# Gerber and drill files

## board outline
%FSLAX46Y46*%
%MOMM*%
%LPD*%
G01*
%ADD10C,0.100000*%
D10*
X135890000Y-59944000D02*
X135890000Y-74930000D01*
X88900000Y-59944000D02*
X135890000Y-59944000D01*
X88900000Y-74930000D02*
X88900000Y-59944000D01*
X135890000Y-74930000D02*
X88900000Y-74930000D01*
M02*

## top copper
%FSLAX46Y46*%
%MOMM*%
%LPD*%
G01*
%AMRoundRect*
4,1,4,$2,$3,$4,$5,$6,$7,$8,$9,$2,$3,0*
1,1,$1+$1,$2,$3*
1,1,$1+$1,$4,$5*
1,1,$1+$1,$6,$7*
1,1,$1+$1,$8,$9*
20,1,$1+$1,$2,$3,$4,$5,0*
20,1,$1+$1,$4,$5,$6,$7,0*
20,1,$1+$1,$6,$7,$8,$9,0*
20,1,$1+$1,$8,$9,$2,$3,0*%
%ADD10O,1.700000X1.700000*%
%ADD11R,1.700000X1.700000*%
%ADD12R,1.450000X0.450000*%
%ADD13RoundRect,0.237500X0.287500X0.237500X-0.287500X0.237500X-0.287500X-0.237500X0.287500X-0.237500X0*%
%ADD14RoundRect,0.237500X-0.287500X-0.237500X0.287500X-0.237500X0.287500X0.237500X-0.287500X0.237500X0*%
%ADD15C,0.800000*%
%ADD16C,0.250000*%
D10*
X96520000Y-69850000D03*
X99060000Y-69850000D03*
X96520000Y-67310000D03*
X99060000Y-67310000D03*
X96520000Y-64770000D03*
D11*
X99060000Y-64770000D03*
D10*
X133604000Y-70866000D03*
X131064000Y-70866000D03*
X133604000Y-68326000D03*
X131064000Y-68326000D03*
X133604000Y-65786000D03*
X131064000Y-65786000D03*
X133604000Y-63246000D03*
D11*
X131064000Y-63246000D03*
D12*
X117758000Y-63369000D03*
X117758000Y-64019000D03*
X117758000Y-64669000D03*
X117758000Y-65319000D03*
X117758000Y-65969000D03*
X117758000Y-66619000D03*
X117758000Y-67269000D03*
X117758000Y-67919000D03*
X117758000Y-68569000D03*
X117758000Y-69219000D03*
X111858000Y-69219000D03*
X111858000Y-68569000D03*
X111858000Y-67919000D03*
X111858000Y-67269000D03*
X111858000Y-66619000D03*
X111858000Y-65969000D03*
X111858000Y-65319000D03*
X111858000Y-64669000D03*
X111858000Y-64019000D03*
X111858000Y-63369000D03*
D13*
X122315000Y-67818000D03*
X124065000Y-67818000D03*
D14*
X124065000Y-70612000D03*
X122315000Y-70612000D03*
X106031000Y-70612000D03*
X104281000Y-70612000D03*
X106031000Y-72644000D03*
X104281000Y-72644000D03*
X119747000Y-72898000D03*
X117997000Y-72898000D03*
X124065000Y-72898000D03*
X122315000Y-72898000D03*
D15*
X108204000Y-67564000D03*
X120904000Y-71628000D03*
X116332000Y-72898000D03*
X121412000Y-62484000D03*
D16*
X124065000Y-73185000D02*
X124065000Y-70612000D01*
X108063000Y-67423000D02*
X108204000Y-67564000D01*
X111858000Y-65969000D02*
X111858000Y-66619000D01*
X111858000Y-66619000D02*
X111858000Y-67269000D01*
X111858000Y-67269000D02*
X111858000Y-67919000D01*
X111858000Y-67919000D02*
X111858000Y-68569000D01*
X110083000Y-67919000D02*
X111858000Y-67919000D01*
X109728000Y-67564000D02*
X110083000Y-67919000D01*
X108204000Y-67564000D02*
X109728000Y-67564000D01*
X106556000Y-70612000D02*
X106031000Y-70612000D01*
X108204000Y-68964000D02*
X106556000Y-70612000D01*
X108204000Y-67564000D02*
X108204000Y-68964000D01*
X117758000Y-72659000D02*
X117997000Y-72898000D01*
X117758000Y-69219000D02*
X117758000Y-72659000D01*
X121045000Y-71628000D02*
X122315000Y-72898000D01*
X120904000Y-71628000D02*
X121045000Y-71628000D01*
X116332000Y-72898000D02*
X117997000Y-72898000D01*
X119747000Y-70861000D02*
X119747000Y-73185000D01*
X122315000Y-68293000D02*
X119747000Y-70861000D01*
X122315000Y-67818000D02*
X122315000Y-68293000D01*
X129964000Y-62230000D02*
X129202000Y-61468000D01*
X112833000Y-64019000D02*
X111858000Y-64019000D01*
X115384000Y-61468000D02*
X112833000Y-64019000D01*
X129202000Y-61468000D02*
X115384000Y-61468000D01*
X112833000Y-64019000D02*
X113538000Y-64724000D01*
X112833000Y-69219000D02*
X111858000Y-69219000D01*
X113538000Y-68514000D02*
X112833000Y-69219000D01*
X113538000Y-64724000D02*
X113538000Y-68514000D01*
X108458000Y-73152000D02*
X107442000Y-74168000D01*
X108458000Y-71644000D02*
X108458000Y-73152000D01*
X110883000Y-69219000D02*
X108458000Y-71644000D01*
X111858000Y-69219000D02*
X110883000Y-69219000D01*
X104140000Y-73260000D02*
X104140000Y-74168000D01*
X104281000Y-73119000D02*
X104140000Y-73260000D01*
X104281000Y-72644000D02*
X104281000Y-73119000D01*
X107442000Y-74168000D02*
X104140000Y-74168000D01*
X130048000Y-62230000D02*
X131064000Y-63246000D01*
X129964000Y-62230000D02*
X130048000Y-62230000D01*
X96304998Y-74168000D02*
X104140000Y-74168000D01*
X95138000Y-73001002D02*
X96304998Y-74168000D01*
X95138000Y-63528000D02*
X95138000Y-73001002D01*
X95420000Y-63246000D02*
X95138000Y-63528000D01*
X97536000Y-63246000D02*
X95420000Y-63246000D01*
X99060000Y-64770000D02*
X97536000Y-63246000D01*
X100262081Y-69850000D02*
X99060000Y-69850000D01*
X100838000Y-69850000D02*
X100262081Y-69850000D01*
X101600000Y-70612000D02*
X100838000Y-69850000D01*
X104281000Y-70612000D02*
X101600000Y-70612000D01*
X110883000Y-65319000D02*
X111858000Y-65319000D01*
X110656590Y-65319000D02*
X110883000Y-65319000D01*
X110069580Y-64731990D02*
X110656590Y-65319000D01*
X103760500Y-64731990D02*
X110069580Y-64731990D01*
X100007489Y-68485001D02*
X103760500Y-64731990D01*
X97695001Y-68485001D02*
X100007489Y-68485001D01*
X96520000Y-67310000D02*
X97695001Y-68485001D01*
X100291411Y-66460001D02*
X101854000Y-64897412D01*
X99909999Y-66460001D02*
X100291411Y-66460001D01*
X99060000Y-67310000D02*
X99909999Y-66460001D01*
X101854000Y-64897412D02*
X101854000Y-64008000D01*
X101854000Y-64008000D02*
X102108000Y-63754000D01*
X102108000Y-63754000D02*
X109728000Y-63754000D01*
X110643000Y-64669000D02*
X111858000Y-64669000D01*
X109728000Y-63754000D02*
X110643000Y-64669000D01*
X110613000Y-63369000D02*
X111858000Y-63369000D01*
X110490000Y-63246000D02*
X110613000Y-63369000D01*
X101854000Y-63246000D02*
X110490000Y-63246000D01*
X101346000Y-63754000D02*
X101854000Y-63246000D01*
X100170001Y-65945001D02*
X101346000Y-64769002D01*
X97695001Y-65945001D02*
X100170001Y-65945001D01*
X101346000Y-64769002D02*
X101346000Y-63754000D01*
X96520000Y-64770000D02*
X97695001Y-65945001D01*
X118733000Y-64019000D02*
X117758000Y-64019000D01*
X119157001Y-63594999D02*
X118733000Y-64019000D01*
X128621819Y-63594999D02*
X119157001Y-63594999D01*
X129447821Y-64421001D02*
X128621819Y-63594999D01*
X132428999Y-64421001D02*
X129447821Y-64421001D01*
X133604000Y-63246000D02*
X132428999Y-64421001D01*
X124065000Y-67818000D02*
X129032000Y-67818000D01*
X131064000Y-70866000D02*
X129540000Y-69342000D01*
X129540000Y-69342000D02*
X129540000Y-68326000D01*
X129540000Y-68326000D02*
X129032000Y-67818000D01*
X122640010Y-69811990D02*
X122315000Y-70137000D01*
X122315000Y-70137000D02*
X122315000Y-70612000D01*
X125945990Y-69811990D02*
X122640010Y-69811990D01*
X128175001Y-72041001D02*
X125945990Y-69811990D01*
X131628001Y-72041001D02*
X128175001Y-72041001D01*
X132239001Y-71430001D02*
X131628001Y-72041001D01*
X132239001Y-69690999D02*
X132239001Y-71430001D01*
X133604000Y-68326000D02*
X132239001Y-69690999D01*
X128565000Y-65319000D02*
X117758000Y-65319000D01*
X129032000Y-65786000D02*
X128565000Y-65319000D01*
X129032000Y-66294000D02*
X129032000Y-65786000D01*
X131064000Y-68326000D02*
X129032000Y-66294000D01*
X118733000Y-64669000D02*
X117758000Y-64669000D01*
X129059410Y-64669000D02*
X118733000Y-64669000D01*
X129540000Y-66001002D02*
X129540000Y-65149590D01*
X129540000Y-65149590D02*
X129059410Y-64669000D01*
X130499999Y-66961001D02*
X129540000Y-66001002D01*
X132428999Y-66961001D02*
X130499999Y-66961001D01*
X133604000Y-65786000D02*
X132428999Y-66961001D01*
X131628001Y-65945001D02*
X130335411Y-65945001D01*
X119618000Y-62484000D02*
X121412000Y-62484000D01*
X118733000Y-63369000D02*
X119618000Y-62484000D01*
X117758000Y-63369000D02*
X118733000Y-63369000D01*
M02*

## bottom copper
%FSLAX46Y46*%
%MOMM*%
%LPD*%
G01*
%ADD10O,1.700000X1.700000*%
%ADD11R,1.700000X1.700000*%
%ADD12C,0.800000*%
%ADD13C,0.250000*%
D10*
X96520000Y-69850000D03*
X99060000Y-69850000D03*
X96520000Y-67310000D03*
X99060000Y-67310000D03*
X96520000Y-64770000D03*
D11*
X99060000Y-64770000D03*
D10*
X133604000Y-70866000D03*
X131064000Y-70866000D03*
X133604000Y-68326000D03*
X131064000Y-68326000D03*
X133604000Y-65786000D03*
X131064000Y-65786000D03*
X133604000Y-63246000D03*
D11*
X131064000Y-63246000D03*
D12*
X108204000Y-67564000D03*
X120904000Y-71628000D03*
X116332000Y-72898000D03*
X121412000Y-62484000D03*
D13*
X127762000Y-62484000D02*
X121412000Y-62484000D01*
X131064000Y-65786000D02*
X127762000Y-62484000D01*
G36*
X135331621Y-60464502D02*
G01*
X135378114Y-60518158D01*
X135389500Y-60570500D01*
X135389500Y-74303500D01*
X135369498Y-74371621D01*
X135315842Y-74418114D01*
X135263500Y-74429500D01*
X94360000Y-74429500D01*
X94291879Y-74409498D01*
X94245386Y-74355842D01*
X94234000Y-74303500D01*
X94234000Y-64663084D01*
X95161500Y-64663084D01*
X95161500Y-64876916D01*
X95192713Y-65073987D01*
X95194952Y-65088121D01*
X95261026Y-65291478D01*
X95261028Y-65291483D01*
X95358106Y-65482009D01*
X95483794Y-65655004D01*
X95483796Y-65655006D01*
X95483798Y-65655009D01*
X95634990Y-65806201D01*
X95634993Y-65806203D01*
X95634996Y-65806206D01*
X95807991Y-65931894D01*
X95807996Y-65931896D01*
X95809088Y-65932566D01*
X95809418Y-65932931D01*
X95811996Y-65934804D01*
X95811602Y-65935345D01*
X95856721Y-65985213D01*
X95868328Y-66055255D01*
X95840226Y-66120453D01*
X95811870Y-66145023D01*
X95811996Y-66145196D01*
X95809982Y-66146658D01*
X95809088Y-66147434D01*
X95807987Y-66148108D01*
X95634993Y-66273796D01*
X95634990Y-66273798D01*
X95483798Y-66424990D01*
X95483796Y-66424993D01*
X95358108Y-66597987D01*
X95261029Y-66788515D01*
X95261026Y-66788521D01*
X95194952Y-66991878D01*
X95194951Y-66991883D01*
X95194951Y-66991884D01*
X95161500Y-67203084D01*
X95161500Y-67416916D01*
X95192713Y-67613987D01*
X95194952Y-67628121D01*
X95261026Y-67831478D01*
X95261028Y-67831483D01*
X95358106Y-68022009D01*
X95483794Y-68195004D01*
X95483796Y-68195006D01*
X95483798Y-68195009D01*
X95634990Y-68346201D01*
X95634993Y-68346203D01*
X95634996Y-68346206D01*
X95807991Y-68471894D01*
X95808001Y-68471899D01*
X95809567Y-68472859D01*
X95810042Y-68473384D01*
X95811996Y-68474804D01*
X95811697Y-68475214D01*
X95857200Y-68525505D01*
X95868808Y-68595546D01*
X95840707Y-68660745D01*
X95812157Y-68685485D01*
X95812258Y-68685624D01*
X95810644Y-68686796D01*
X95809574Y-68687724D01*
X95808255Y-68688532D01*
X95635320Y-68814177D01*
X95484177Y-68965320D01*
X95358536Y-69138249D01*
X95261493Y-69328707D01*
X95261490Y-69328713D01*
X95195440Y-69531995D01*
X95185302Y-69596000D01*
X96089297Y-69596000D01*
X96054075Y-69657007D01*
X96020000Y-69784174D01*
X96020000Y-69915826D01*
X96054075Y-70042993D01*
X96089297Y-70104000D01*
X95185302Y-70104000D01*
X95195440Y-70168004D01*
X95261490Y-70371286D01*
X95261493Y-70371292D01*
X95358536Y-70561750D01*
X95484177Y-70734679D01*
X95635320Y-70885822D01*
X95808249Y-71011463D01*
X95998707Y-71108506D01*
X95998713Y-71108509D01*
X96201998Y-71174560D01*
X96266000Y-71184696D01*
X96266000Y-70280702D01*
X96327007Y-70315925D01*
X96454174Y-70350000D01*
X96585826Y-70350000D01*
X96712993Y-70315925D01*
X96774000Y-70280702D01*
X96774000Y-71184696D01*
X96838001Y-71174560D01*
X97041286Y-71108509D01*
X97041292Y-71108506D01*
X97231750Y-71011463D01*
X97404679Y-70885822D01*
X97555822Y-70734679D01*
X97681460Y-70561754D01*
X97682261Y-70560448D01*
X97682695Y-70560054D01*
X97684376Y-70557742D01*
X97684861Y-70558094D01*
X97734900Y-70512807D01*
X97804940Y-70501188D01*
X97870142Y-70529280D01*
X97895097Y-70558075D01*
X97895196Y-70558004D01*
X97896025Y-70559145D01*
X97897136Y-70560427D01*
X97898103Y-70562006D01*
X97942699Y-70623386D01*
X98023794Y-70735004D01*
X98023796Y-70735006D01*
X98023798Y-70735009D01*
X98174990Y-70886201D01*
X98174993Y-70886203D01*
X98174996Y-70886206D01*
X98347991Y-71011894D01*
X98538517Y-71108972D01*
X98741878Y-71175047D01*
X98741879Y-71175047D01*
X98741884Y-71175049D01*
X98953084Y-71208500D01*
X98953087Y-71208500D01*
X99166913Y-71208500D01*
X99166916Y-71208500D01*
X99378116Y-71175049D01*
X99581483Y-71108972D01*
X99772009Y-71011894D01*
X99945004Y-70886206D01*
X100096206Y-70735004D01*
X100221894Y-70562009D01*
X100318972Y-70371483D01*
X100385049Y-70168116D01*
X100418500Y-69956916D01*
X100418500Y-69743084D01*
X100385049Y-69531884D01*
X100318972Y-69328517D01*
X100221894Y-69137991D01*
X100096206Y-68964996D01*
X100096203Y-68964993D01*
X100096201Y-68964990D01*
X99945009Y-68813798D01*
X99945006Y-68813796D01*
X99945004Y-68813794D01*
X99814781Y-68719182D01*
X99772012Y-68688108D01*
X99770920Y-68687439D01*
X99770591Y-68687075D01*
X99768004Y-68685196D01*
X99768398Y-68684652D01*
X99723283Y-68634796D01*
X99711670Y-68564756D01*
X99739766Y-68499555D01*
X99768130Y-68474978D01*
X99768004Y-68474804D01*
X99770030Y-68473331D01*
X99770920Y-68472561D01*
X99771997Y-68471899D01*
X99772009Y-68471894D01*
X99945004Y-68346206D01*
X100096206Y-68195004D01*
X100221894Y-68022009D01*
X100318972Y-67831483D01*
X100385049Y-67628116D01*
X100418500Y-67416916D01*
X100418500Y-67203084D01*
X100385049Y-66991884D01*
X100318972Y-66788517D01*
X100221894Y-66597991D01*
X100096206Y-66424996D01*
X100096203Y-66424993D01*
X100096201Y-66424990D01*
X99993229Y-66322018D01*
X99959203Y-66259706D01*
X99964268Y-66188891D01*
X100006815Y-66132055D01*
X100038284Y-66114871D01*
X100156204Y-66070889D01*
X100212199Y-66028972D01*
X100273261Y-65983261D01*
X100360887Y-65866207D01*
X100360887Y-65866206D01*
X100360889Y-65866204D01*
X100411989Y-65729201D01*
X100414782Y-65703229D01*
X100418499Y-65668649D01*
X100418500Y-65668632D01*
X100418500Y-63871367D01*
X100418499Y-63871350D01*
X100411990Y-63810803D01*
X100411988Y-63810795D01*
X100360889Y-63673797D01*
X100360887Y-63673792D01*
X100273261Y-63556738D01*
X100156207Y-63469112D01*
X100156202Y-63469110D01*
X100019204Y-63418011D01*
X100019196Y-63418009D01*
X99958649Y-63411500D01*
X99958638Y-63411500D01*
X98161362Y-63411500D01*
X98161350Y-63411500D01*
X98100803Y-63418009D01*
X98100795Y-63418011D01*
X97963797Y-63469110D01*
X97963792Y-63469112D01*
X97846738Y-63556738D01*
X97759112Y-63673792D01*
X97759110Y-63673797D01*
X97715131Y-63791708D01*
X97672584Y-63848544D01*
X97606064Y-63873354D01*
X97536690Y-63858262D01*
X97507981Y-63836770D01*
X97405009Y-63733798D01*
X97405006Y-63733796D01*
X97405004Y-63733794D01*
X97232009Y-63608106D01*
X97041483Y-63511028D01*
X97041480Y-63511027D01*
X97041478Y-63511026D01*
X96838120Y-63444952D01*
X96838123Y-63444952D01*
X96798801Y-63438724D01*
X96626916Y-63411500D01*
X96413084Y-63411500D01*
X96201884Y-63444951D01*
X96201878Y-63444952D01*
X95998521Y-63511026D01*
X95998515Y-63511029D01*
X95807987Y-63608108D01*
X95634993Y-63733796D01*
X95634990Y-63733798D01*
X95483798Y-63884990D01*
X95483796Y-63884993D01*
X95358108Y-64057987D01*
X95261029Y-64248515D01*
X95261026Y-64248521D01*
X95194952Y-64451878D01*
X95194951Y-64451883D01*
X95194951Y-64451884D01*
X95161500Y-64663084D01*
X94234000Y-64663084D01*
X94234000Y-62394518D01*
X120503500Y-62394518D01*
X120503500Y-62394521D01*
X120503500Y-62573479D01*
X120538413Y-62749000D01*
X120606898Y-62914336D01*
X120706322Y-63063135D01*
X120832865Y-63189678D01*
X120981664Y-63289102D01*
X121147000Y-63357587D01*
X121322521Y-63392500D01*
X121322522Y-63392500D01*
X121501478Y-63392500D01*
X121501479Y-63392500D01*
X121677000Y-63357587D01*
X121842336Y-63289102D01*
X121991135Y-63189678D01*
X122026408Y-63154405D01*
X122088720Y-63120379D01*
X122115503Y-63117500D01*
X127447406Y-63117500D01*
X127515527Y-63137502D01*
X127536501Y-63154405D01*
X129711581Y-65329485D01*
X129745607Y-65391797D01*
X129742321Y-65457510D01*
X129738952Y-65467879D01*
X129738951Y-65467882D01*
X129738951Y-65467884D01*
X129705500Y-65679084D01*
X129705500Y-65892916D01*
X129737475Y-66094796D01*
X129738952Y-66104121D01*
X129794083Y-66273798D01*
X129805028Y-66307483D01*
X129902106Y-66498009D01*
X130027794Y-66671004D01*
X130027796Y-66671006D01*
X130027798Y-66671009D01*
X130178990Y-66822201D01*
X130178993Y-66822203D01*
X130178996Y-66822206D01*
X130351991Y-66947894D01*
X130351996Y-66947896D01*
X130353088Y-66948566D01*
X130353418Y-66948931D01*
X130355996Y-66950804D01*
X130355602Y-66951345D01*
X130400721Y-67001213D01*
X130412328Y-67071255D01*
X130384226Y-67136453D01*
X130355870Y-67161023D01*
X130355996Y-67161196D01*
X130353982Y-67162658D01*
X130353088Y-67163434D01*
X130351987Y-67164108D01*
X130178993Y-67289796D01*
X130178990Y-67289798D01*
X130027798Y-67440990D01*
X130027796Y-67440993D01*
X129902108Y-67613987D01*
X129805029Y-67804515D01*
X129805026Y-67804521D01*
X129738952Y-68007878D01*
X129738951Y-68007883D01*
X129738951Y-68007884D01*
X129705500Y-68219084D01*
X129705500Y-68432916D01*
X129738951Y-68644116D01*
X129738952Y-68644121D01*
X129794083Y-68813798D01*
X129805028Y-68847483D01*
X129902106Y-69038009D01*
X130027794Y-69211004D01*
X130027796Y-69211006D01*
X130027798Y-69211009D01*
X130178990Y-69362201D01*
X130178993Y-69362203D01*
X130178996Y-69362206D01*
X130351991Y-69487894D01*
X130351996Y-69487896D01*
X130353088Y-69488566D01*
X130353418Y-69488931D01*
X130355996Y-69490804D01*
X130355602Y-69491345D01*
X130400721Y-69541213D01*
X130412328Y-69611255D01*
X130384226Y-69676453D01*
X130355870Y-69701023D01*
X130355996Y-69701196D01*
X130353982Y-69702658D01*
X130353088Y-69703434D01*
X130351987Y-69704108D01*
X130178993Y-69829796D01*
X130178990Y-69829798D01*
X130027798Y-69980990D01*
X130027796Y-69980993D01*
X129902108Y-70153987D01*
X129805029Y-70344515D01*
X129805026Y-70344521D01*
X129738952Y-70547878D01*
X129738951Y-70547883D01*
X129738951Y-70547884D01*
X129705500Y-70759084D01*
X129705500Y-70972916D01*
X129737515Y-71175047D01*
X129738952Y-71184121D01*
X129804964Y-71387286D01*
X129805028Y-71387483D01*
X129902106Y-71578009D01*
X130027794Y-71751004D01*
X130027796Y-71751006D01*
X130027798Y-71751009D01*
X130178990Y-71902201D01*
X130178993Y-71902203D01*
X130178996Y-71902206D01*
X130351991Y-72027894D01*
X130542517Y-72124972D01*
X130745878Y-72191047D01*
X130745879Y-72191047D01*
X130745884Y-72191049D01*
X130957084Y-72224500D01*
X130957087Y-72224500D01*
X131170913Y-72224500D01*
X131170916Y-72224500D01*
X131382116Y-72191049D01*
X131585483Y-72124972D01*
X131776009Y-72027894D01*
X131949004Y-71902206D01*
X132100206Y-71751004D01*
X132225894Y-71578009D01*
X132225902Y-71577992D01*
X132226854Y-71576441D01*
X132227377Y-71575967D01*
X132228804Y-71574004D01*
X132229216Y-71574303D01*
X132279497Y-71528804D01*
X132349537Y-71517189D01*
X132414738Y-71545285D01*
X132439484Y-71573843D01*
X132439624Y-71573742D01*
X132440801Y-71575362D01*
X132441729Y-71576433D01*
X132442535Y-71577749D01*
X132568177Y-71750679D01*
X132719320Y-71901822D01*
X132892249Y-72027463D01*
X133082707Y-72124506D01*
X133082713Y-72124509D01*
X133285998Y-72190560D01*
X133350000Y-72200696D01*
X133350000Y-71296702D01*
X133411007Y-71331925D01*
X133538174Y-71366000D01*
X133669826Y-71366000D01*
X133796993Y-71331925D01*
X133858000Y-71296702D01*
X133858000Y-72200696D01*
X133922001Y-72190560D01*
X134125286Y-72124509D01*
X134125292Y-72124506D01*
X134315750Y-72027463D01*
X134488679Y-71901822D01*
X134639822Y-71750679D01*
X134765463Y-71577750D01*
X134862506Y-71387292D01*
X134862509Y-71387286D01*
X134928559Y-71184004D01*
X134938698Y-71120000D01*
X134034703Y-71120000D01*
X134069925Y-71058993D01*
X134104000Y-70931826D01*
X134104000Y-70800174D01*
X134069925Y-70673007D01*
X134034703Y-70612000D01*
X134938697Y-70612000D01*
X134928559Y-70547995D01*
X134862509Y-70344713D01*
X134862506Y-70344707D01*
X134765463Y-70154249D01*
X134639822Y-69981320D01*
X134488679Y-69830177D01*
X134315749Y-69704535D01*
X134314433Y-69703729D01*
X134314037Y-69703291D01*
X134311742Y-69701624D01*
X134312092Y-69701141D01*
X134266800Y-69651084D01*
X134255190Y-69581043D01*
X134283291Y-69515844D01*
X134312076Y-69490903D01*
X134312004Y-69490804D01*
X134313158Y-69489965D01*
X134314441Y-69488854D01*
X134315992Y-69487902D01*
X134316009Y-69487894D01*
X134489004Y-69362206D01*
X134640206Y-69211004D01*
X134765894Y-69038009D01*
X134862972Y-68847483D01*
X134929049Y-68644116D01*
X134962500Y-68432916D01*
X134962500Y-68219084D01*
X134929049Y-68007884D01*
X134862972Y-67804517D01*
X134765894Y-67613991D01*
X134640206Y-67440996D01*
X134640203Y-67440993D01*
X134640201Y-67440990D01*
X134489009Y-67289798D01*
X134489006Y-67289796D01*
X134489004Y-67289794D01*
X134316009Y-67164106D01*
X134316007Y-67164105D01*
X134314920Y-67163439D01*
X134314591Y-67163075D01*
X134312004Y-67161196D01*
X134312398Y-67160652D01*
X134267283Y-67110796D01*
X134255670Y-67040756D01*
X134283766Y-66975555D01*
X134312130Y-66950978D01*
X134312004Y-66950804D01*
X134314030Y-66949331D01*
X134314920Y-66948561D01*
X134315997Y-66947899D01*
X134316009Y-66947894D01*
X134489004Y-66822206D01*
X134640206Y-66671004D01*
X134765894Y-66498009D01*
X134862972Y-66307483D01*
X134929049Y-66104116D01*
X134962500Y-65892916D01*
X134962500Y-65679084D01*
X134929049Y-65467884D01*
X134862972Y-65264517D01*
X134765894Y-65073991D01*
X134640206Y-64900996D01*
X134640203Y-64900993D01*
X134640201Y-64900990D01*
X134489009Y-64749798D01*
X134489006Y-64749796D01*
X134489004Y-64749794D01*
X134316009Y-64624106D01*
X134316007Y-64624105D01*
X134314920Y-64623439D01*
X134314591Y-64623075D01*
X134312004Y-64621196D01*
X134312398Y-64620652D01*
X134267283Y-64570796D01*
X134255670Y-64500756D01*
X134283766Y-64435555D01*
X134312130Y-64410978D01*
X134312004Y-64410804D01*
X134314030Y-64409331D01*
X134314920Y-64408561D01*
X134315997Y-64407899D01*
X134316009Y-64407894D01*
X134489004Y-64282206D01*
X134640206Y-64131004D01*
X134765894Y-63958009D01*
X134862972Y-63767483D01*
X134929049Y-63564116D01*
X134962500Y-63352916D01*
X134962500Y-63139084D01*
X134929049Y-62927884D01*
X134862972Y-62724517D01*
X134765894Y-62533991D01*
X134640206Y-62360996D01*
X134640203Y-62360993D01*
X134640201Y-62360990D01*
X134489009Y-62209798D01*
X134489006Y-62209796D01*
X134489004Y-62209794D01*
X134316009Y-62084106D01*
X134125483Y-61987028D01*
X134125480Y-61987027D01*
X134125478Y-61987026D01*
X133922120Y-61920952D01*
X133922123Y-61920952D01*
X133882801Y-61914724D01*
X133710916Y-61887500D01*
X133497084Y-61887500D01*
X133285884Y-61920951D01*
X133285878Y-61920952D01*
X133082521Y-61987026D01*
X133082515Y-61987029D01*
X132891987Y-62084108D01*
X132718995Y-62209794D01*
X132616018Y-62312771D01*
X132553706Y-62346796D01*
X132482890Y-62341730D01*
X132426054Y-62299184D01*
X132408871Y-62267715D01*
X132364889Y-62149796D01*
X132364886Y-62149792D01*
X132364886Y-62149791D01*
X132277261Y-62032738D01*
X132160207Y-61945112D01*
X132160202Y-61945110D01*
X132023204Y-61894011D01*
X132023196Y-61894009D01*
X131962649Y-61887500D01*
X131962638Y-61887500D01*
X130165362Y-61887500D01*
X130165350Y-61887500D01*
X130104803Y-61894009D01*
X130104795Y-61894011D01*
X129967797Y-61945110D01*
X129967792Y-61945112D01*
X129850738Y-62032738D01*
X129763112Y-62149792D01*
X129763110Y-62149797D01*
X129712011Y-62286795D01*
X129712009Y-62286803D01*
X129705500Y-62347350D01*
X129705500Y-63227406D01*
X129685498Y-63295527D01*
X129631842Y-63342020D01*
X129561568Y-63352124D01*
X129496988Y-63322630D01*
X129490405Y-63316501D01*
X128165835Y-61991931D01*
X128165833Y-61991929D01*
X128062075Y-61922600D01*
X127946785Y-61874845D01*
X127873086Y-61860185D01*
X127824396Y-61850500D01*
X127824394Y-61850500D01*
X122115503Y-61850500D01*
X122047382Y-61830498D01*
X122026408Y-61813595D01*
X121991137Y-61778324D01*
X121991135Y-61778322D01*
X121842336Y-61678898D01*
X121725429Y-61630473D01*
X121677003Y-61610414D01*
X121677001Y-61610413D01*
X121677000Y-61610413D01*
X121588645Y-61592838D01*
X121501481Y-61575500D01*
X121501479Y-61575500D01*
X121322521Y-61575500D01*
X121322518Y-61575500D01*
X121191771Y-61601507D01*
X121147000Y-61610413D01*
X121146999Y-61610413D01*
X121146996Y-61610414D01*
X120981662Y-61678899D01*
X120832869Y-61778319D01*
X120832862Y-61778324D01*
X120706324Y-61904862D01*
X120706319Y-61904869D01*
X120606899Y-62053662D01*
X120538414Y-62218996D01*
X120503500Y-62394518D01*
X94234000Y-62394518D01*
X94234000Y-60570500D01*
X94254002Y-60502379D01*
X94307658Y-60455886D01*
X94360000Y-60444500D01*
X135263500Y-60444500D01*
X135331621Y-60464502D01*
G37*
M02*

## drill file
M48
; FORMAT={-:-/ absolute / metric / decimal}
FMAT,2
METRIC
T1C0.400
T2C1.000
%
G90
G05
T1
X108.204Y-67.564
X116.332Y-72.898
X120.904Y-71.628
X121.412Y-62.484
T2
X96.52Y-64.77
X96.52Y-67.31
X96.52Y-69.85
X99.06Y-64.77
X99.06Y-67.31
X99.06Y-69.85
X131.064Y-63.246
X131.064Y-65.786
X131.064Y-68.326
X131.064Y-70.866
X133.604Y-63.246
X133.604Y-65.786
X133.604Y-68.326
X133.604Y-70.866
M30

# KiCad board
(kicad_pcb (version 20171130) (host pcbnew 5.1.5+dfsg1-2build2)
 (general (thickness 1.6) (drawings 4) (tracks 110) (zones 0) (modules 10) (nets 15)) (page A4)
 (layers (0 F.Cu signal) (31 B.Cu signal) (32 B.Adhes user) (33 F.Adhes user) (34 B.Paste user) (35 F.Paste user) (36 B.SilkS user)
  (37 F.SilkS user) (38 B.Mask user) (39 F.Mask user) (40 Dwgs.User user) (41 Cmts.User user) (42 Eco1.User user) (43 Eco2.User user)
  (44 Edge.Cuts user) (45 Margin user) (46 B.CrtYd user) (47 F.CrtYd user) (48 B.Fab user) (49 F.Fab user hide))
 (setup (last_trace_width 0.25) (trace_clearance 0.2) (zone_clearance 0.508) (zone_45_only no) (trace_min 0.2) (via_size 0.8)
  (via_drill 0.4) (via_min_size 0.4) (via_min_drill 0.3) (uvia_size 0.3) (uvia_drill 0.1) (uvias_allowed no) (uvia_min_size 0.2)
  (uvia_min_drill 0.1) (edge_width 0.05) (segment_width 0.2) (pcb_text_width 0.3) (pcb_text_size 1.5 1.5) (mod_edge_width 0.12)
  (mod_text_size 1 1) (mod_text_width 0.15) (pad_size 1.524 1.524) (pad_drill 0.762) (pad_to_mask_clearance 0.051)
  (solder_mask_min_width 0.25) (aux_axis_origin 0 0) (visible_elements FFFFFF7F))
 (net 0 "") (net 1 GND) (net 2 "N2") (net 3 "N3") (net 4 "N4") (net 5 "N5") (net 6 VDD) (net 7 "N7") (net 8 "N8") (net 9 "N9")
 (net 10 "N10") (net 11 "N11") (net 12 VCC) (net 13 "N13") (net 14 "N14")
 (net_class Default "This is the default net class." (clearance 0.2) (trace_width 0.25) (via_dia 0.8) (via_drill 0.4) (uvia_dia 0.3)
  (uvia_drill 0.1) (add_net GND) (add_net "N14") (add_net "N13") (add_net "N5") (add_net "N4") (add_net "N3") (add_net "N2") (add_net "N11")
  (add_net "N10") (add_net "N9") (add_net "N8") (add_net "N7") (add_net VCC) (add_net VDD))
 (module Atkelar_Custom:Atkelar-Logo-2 (layer F.Cu) (at 105.41 65.024 90)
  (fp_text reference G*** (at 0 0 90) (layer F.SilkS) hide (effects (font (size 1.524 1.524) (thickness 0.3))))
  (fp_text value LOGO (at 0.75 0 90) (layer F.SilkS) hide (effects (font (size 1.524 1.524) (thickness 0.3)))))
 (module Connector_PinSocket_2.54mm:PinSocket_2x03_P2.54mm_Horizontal (layer F.Cu) (at 99.06 64.77)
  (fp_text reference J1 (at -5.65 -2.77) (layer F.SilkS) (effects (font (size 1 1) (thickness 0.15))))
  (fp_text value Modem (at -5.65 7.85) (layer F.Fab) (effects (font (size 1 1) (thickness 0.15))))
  (pad 6 thru_hole oval (at -2.54 5.08) (size 1.7 1.7) (drill 1) (layers *.Cu *.Mask) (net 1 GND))
  (pad 5 thru_hole oval (at 0 5.08) (size 1.7 1.7) (drill 1) (layers *.Cu *.Mask) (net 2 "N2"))
  (pad 4 thru_hole oval (at -2.54 2.54) (size 1.7 1.7) (drill 1) (layers *.Cu *.Mask) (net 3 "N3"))
  (pad 3 thru_hole oval (at 0 2.54) (size 1.7 1.7) (drill 1) (layers *.Cu *.Mask) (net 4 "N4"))
  (pad 2 thru_hole oval (at -2.54 0) (size 1.7 1.7) (drill 1) (layers *.Cu *.Mask) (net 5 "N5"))
  (pad 1 thru_hole rect (at 0 0) (size 1.7 1.7) (drill 1) (layers *.Cu *.Mask) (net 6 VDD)))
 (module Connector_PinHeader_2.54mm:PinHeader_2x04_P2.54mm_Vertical (layer F.Cu) (at 131.064 63.246)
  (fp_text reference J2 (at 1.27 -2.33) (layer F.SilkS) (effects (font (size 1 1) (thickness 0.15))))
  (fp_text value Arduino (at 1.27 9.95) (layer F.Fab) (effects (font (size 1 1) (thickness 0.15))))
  (pad 8 thru_hole oval (at 2.54 7.62) (size 1.7 1.7) (drill 1) (layers *.Cu *.Mask) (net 1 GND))
  (pad 7 thru_hole oval (at 0 7.62) (size 1.7 1.7) (drill 1) (layers *.Cu *.Mask) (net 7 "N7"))
  (pad 6 thru_hole oval (at 2.54 5.08) (size 1.7 1.7) (drill 1) (layers *.Cu *.Mask) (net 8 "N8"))
  (pad 5 thru_hole oval (at 0 5.08) (size 1.7 1.7) (drill 1) (layers *.Cu *.Mask) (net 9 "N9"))
  (pad 4 thru_hole oval (at 2.54 2.54) (size 1.7 1.7) (drill 1) (layers *.Cu *.Mask) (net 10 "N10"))
  (pad 3 thru_hole oval (at 0 2.54) (size 1.7 1.7) (drill 1) (layers *.Cu *.Mask) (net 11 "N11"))
  (pad 2 thru_hole oval (at 2.54 0) (size 1.7 1.7) (drill 1) (layers *.Cu *.Mask) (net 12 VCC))
  (pad 1 thru_hole rect (at 0 0) (size 1.7 1.7) (drill 1) (layers *.Cu *.Mask) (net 6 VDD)))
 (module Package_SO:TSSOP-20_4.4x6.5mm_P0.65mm (layer F.Cu) (at 114.808 66.294)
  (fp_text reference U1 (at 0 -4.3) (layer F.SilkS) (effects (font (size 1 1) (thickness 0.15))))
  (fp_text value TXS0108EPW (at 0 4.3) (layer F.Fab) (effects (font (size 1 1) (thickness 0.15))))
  (pad 20 smd rect (at 2.95 -2.925) (size 1.45 0.45) (layers F.Cu F.Paste F.Mask) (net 11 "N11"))
  (pad 19 smd rect (at 2.95 -2.275) (size 1.45 0.45) (layers F.Cu F.Paste F.Mask) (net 12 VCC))
  (pad 18 smd rect (at 2.95 -1.625) (size 1.45 0.45) (layers F.Cu F.Paste F.Mask) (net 10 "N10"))
  (pad 17 smd rect (at 2.95 -0.975) (size 1.45 0.45) (layers F.Cu F.Paste F.Mask) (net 9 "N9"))
  (pad 16 smd rect (at 2.95 -0.325) (size 1.45 0.45) (layers F.Cu F.Paste F.Mask))
  (pad 15 smd rect (at 2.95 0.325) (size 1.45 0.45) (layers F.Cu F.Paste F.Mask))
  (pad 14 smd rect (at 2.95 0.975) (size 1.45 0.45) (layers F.Cu F.Paste F.Mask))
  (pad 13 smd rect (at 2.95 1.625) (size 1.45 0.45) (layers F.Cu F.Paste F.Mask))
  (pad 12 smd rect (at 2.95 2.275) (size 1.45 0.45) (layers F.Cu F.Paste F.Mask))
  (pad 11 smd rect (at 2.95 2.925) (size 1.45 0.45) (layers F.Cu F.Paste F.Mask) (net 1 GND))
  (pad 10 smd rect (at -2.95 2.925) (size 1.45 0.45) (layers F.Cu F.Paste F.Mask) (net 6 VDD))
  (pad 9 smd rect (at -2.95 2.275) (size 1.45 0.45) (layers F.Cu F.Paste F.Mask) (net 1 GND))
  (pad 8 smd rect (at -2.95 1.625) (size 1.45 0.45) (layers F.Cu F.Paste F.Mask) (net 1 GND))
  (pad 7 smd rect (at -2.95 0.975) (size 1.45 0.45) (layers F.Cu F.Paste F.Mask) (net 1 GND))
  (pad 6 smd rect (at -2.95 0.325) (size 1.45 0.45) (layers F.Cu F.Paste F.Mask) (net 1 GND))
  (pad 5 smd rect (at -2.95 -0.325) (size 1.45 0.45) (layers F.Cu F.Paste F.Mask) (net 1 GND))
  (pad 4 smd rect (at -2.95 -0.975) (size 1.45 0.45) (layers F.Cu F.Paste F.Mask) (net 3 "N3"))
  (pad 3 smd rect (at -2.95 -1.625) (size 1.45 0.45) (layers F.Cu F.Paste F.Mask) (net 4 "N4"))
  (pad 2 smd rect (at -2.95 -2.275) (size 1.45 0.45) (layers F.Cu F.Paste F.Mask) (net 6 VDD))
  (pad 1 smd rect (at -2.95 -2.925) (size 1.45 0.45) (layers F.Cu F.Paste F.Mask) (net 5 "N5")))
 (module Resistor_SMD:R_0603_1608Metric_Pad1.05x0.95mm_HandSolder (layer F.Cu) (at 123.19 67.818 180)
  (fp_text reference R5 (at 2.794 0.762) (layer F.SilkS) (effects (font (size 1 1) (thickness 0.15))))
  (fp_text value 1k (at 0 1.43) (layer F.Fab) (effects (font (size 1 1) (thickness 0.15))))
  (pad 2 smd roundrect (at 0.875 0 180) (size 1.05 0.95) (layers F.Cu F.Paste F.Mask) (roundrect_rratio 0.25) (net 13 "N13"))
  (pad 1 smd roundrect (at -0.875 0 180) (size 1.05 0.95) (layers F.Cu F.Paste F.Mask) (roundrect_rratio 0.25) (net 7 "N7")))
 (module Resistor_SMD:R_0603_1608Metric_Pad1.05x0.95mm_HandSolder (layer F.Cu) (at 123.19 70.612)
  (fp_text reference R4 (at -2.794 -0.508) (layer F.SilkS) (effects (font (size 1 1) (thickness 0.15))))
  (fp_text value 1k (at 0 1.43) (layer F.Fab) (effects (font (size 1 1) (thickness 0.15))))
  (pad 2 smd roundrect (at 0.875 0) (size 1.05 0.95) (layers F.Cu F.Paste F.Mask) (roundrect_rratio 0.25) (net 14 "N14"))
  (pad 1 smd roundrect (at -0.875 0) (size 1.05 0.95) (layers F.Cu F.Paste F.Mask) (roundrect_rratio 0.25) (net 8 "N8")))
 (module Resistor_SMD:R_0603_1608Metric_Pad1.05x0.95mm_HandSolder (layer F.Cu) (at 105.156 70.612)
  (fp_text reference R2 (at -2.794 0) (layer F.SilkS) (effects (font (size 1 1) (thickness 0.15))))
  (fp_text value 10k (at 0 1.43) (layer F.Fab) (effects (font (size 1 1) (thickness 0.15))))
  (pad 2 smd roundrect (at 0.875 0) (size 1.05 0.95) (layers F.Cu F.Paste F.Mask) (roundrect_rratio 0.25) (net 1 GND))
  (pad 1 smd roundrect (at -0.875 0) (size 1.05 0.95) (layers F.Cu F.Paste F.Mask) (roundrect_rratio 0.25) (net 2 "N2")))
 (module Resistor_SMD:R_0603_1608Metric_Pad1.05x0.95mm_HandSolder (layer F.Cu) (at 105.156 72.644)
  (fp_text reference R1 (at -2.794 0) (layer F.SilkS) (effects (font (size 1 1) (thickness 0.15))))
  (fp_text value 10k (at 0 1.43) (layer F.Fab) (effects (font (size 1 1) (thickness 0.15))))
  (pad 2 smd roundrect (at 0.875 0) (size 1.05 0.95) (layers F.Cu F.Paste F.Mask) (roundrect_rratio 0.25))
  (pad 1 smd roundrect (at -0.875 0) (size 1.05 0.95) (layers F.Cu F.Paste F.Mask) (roundrect_rratio 0.25) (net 6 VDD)))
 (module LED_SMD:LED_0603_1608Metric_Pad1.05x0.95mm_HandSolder (layer F.Cu) (at 118.872 72.898)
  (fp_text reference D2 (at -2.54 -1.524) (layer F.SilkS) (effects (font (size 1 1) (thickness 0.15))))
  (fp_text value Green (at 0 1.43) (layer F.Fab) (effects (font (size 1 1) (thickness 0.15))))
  (pad 2 smd roundrect (at 0.875 0) (size 1.05 0.95) (layers F.Cu F.Paste F.Mask) (roundrect_rratio 0.25) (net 13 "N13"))
  (pad 1 smd roundrect (at -0.875 0) (size 1.05 0.95) (layers F.Cu F.Paste F.Mask) (roundrect_rratio 0.25) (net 1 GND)))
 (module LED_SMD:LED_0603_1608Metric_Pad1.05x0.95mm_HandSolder (layer F.Cu) (at 123.19 72.898)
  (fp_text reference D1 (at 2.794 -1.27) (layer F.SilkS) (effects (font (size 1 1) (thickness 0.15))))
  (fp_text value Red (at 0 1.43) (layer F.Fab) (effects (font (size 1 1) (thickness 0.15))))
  (pad 2 smd roundrect (at 0.875 0) (size 1.05 0.95) (layers F.Cu F.Paste F.Mask) (roundrect_rratio 0.25) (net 14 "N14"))
  (pad 1 smd roundrect (at -0.875 0) (size 1.05 0.95) (layers F.Cu F.Paste F.Mask) (roundrect_rratio 0.25) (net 1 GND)))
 (gr_line (start 135.89 59.944) (end 135.89 74.93) (layer Edge.Cuts) (width 0.1))
 (gr_line (start 88.9 59.944) (end 135.89 59.944) (layer Edge.Cuts) (width 0.1))
 (gr_line (start 88.9 74.93) (end 88.9 59.944) (layer Edge.Cuts) (width 0.1))
 (gr_line (start 135.89 74.93) (end 88.9 74.93) (layer Edge.Cuts) (width 0.1))
 (segment (start 124.065 73.185) (end 124.065 70.612) (width 0.25) (layer F.Cu) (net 14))
 (via (at 108.204 67.564) (size 0.8) (drill 0.4) (layers F.Cu B.Cu) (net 1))
 (segment (start 108.063 67.423) (end 108.204 67.564) (width 0.25) (layer F.Cu) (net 1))
 (via (at 120.904 71.628) (size 0.8) (drill 0.4) (layers F.Cu B.Cu) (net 1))
 (segment (start 111.858 65.969) (end 111.858 66.619) (width 0.25) (layer F.Cu) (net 1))
 (segment (start 111.858 66.619) (end 111.858 67.269) (width 0.25) (layer F.Cu) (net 1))
 (segment (start 111.858 67.269) (end 111.858 67.919) (width 0.25) (layer F.Cu) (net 1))
 (segment (start 111.858 67.919) (end 111.858 68.569) (width 0.25) (layer F.Cu) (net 1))
 (segment (start 110.083 67.919) (end 111.858 67.919) (width 0.25) (layer F.Cu) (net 1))
 (segment (start 109.728 67.564) (end 110.083 67.919) (width 0.25) (layer F.Cu) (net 1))
 (segment (start 108.204 67.564) (end 109.728 67.564) (width 0.25) (layer F.Cu) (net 1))
 (segment (start 106.556 70.612) (end 106.031 70.612) (width 0.25) (layer F.Cu) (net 1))
 (segment (start 108.204 68.964) (end 106.556 70.612) (width 0.25) (layer F.Cu) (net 1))
 (segment (start 108.204 67.564) (end 108.204 68.964) (width 0.25) (layer F.Cu) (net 1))
 (segment (start 117.758 72.659) (end 117.997 72.898) (width 0.25) (layer F.Cu) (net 1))
 (segment (start 117.758 69.219) (end 117.758 72.659) (width 0.25) (layer F.Cu) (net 1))
 (segment (start 121.045 71.628) (end 122.315 72.898) (width 0.25) (layer F.Cu) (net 1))
 (segment (start 120.904 71.628) (end 121.045 71.628) (width 0.25) (layer F.Cu) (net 1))
 (via (at 116.332 72.898) (size 0.8) (drill 0.4) (layers F.Cu B.Cu) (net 1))
 (segment (start 116.332 72.898) (end 117.997 72.898) (width 0.25) (layer F.Cu) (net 1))
 (segment (start 119.747 70.861) (end 119.747 73.185) (width 0.25) (layer F.Cu) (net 13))
 (segment (start 122.315 68.293) (end 119.747 70.861) (width 0.25) (layer F.Cu) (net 13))
 (segment (start 122.315 67.818) (end 122.315 68.293) (width 0.25) (layer F.Cu) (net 13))
 (segment (start 129.964 62.23) (end 129.202 61.468) (width 0.25) (layer F.Cu) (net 6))
 (segment (start 112.833 64.019) (end 111.858 64.019) (width 0.25) (layer F.Cu) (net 6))
 (segment (start 115.384 61.468) (end 112.833 64.019) (width 0.25) (layer F.Cu) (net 6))
 (segment (start 129.202 61.468) (end 115.384 61.468) (width 0.25) (layer F.Cu) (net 6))
 (segment (start 112.833 64.019) (end 113.538 64.724) (width 0.25) (layer F.Cu) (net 6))
 (segment (start 112.833 69.219) (end 111.858 69.219) (width 0.25) (layer F.Cu) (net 6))
 (segment (start 113.538 68.514) (end 112.833 69.219) (width 0.25) (layer F.Cu) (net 6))
 (segment (start 113.538 64.724) (end 113.538 68.514) (width 0.25) (layer F.Cu) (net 6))
 (segment (start 108.458 73.152) (end 107.442 74.168) (width 0.25) (layer F.Cu) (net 6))
 (segment (start 108.458 71.644) (end 108.458 73.152) (width 0.25) (layer F.Cu) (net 6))
 (segment (start 110.883 69.219) (end 108.458 71.644) (width 0.25) (layer F.Cu) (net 6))
 (segment (start 111.858 69.219) (end 110.883 69.219) (width 0.25) (layer F.Cu) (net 6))
 (segment (start 104.14 73.26) (end 104.14 74.168) (width 0.25) (layer F.Cu) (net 6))
 (segment (start 104.281 73.119) (end 104.14 73.26) (width 0.25) (layer F.Cu) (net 6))
 (segment (start 104.281 72.644) (end 104.281 73.119) (width 0.25) (layer F.Cu) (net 6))
 (segment (start 107.442 74.168) (end 104.14 74.168) (width 0.25) (layer F.Cu) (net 6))
 (segment (start 130.048 62.23) (end 131.064 63.246) (width 0.25) (layer F.Cu) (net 6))
 (segment (start 129.964 62.23) (end 130.048 62.23) (width 0.25) (layer F.Cu) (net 6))
 (segment (start 96.304998 74.168) (end 104.14 74.168) (width 0.25) (layer F.Cu) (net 6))
 (segment (start 95.138 73.001002) (end 96.304998 74.168) (width 0.25) (layer F.Cu) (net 6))
 (segment (start 95.138 63.528) (end 95.138 73.001002) (width 0.25) (layer F.Cu) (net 6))
 (segment (start 95.42 63.246) (end 95.138 63.528) (width 0.25) (layer F.Cu) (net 6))
 (segment (start 97.536 63.246) (end 95.42 63.246) (width 0.25) (layer F.Cu) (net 6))
 (segment (start 99.06 64.77) (end 97.536 63.246) (width 0.25) (layer F.Cu) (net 6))
 (segment (start 100.262081 69.85) (end 99.06 69.85) (width 0.25) (layer F.Cu) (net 2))
 (segment (start 100.838 69.85) (end 100.262081 69.85) (width 0.25) (layer F.Cu) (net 2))
 (segment (start 101.6 70.612) (end 100.838 69.85) (width 0.25) (layer F.Cu) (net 2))
 (segment (start 104.281 70.612) (end 101.6 70.612) (width 0.25) (layer F.Cu) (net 2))
 (segment (start 110.883 65.319) (end 111.858 65.319) (width 0.25) (layer F.Cu) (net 3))
 (segment (start 110.65659 65.319) (end 110.883 65.319) (width 0.25) (layer F.Cu) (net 3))
 (segment (start 110.06958 64.73199) (end 110.65659 65.319) (width 0.25) (layer F.Cu) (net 3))
 (segment (start 103.7605 64.73199) (end 110.06958 64.73199) (width 0.25) (layer F.Cu) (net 3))
 (segment (start 100.007489 68.485001) (end 103.7605 64.73199) (width 0.25) (layer F.Cu) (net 3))
 (segment (start 97.695001 68.485001) (end 100.007489 68.485001) (width 0.25) (layer F.Cu) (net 3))
 (segment (start 96.52 67.31) (end 97.695001 68.485001) (width 0.25) (layer F.Cu) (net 3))
 (segment (start 100.291411 66.460001) (end 101.854 64.897412) (width 0.25) (layer F.Cu) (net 4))
 (segment (start 99.909999 66.460001) (end 100.291411 66.460001) (width 0.25) (layer F.Cu) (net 4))
 (segment (start 99.06 67.31) (end 99.909999 66.460001) (width 0.25) (layer F.Cu) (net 4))
 (segment (start 101.854 64.897412) (end 101.854 64.008) (width 0.25) (layer F.Cu) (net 4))
 (segment (start 101.854 64.008) (end 102.108 63.754) (width 0.25) (layer F.Cu) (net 4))
 (segment (start 102.108 63.754) (end 109.728 63.754) (width 0.25) (layer F.Cu) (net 4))
 (segment (start 110.643 64.669) (end 111.858 64.669) (width 0.25) (layer F.Cu) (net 4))
 (segment (start 109.728 63.754) (end 110.643 64.669) (width 0.25) (layer F.Cu) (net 4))
 (segment (start 110.613 63.369) (end 111.858 63.369) (width 0.25) (layer F.Cu) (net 5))
 (segment (start 110.49 63.246) (end 110.613 63.369) (width 0.25) (layer F.Cu) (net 5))
 (segment (start 101.854 63.246) (end 110.49 63.246) (width 0.25) (layer F.Cu) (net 5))
 (segment (start 101.346 63.754) (end 101.854 63.246) (width 0.25) (layer F.Cu) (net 5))
 (segment (start 100.170001 65.945001) (end 101.346 64.769002) (width 0.25) (layer F.Cu) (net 5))
 (segment (start 97.695001 65.945001) (end 100.170001 65.945001) (width 0.25) (layer F.Cu) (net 5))
 (segment (start 101.346 64.769002) (end 101.346 63.754) (width 0.25) (layer F.Cu) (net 5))
 (segment (start 96.52 64.77) (end 97.695001 65.945001) (width 0.25) (layer F.Cu) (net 5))
 (segment (start 118.733 64.019) (end 117.758 64.019) (width 0.25) (layer F.Cu) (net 12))
 (segment (start 119.157001 63.594999) (end 118.733 64.019) (width 0.25) (layer F.Cu) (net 12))
 (segment (start 128.621819 63.594999) (end 119.157001 63.594999) (width 0.25) (layer F.Cu) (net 12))
 (segment (start 129.447821 64.421001) (end 128.621819 63.594999) (width 0.25) (layer F.Cu) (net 12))
 (segment (start 132.428999 64.421001) (end 129.447821 64.421001) (width 0.25) (layer F.Cu) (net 12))
 (segment (start 133.604 63.246) (end 132.428999 64.421001) (width 0.25) (layer F.Cu) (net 12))
 (segment (start 124.065 67.818) (end 129.032 67.818) (width 0.25) (layer F.Cu) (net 7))
 (segment (start 131.064 70.866) (end 129.54 69.342) (width 0.25) (layer F.Cu) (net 7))
 (segment (start 129.54 69.342) (end 129.54 68.326) (width 0.25) (layer F.Cu) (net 7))
 (segment (start 129.54 68.326) (end 129.032 67.818) (width 0.25) (layer F.Cu) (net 7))
 (segment (start 122.64001 69.81199) (end 122.315 70.137) (width 0.25) (layer F.Cu) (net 8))
 (segment (start 122.315 70.137) (end 122.315 70.612) (width 0.25) (layer F.Cu) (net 8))
 (segment (start 125.94599 69.81199) (end 122.64001 69.81199) (width 0.25) (layer F.Cu) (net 8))
 (segment (start 128.175001 72.041001) (end 125.94599 69.81199) (width 0.25) (layer F.Cu) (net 8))
 (segment (start 131.628001 72.041001) (end 128.175001 72.041001) (width 0.25) (layer F.Cu) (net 8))
 (segment (start 132.239001 71.430001) (end 131.628001 72.041001) (width 0.25) (layer F.Cu) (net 8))
 (segment (start 132.239001 69.690999) (end 132.239001 71.430001) (width 0.25) (layer F.Cu) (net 8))
 (segment (start 133.604 68.326) (end 132.239001 69.690999) (width 0.25) (layer F.Cu) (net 8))
 (segment (start 128.565 65.319) (end 117.758 65.319) (width 0.25) (layer F.Cu) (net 9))
 (segment (start 129.032 65.786) (end 128.565 65.319) (width 0.25) (layer F.Cu) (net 9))
 (segment (start 129.032 66.294) (end 129.032 65.786) (width 0.25) (layer F.Cu) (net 9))
 (segment (start 131.064 68.326) (end 129.032 66.294) (width 0.25) (layer F.Cu) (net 9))
 (segment (start 118.733 64.669) (end 117.758 64.669) (width 0.25) (layer F.Cu) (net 10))
 (segment (start 129.05941 64.669) (end 118.733 64.669) (width 0.25) (layer F.Cu) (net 10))
 (segment (start 129.54 66.001002) (end 129.54 65.14959) (width 0.25) (layer F.Cu) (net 10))
 (segment (start 129.54 65.14959) (end 129.05941 64.669) (width 0.25) (layer F.Cu) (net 10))
 (segment (start 130.499999 66.961001) (end 129.54 66.001002) (width 0.25) (layer F.Cu) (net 10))
 (segment (start 132.428999 66.961001) (end 130.499999 66.961001) (width 0.25) (layer F.Cu) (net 10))
 (segment (start 133.604 65.786) (end 132.428999 66.961001) (width 0.25) (layer F.Cu) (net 10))
 (segment (start 131.628001 65.945001) (end 130.335411 65.945001) (width 0.25) (layer F.Cu) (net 11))
 (via (at 121.412 62.484) (size 0.8) (drill 0.4) (layers F.Cu B.Cu) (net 11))
 (segment (start 119.618 62.484) (end 121.412 62.484) (width 0.25) (layer F.Cu) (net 11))
 (segment (start 118.733 63.369) (end 119.618 62.484) (width 0.25) (layer F.Cu) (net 11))
 (segment (start 117.758 63.369) (end 118.733 63.369) (width 0.25) (layer F.Cu) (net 11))
 (segment (start 127.762 62.484) (end 121.412 62.484) (width 0.25) (layer B.Cu) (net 11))
 (segment (start 131.064 65.786) (end 127.762 62.484) (width 0.25) (layer B.Cu) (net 11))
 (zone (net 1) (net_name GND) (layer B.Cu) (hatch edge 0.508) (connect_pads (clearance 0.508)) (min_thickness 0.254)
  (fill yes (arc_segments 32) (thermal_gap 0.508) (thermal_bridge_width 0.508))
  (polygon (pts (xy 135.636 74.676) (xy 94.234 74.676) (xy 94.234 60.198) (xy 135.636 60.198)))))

